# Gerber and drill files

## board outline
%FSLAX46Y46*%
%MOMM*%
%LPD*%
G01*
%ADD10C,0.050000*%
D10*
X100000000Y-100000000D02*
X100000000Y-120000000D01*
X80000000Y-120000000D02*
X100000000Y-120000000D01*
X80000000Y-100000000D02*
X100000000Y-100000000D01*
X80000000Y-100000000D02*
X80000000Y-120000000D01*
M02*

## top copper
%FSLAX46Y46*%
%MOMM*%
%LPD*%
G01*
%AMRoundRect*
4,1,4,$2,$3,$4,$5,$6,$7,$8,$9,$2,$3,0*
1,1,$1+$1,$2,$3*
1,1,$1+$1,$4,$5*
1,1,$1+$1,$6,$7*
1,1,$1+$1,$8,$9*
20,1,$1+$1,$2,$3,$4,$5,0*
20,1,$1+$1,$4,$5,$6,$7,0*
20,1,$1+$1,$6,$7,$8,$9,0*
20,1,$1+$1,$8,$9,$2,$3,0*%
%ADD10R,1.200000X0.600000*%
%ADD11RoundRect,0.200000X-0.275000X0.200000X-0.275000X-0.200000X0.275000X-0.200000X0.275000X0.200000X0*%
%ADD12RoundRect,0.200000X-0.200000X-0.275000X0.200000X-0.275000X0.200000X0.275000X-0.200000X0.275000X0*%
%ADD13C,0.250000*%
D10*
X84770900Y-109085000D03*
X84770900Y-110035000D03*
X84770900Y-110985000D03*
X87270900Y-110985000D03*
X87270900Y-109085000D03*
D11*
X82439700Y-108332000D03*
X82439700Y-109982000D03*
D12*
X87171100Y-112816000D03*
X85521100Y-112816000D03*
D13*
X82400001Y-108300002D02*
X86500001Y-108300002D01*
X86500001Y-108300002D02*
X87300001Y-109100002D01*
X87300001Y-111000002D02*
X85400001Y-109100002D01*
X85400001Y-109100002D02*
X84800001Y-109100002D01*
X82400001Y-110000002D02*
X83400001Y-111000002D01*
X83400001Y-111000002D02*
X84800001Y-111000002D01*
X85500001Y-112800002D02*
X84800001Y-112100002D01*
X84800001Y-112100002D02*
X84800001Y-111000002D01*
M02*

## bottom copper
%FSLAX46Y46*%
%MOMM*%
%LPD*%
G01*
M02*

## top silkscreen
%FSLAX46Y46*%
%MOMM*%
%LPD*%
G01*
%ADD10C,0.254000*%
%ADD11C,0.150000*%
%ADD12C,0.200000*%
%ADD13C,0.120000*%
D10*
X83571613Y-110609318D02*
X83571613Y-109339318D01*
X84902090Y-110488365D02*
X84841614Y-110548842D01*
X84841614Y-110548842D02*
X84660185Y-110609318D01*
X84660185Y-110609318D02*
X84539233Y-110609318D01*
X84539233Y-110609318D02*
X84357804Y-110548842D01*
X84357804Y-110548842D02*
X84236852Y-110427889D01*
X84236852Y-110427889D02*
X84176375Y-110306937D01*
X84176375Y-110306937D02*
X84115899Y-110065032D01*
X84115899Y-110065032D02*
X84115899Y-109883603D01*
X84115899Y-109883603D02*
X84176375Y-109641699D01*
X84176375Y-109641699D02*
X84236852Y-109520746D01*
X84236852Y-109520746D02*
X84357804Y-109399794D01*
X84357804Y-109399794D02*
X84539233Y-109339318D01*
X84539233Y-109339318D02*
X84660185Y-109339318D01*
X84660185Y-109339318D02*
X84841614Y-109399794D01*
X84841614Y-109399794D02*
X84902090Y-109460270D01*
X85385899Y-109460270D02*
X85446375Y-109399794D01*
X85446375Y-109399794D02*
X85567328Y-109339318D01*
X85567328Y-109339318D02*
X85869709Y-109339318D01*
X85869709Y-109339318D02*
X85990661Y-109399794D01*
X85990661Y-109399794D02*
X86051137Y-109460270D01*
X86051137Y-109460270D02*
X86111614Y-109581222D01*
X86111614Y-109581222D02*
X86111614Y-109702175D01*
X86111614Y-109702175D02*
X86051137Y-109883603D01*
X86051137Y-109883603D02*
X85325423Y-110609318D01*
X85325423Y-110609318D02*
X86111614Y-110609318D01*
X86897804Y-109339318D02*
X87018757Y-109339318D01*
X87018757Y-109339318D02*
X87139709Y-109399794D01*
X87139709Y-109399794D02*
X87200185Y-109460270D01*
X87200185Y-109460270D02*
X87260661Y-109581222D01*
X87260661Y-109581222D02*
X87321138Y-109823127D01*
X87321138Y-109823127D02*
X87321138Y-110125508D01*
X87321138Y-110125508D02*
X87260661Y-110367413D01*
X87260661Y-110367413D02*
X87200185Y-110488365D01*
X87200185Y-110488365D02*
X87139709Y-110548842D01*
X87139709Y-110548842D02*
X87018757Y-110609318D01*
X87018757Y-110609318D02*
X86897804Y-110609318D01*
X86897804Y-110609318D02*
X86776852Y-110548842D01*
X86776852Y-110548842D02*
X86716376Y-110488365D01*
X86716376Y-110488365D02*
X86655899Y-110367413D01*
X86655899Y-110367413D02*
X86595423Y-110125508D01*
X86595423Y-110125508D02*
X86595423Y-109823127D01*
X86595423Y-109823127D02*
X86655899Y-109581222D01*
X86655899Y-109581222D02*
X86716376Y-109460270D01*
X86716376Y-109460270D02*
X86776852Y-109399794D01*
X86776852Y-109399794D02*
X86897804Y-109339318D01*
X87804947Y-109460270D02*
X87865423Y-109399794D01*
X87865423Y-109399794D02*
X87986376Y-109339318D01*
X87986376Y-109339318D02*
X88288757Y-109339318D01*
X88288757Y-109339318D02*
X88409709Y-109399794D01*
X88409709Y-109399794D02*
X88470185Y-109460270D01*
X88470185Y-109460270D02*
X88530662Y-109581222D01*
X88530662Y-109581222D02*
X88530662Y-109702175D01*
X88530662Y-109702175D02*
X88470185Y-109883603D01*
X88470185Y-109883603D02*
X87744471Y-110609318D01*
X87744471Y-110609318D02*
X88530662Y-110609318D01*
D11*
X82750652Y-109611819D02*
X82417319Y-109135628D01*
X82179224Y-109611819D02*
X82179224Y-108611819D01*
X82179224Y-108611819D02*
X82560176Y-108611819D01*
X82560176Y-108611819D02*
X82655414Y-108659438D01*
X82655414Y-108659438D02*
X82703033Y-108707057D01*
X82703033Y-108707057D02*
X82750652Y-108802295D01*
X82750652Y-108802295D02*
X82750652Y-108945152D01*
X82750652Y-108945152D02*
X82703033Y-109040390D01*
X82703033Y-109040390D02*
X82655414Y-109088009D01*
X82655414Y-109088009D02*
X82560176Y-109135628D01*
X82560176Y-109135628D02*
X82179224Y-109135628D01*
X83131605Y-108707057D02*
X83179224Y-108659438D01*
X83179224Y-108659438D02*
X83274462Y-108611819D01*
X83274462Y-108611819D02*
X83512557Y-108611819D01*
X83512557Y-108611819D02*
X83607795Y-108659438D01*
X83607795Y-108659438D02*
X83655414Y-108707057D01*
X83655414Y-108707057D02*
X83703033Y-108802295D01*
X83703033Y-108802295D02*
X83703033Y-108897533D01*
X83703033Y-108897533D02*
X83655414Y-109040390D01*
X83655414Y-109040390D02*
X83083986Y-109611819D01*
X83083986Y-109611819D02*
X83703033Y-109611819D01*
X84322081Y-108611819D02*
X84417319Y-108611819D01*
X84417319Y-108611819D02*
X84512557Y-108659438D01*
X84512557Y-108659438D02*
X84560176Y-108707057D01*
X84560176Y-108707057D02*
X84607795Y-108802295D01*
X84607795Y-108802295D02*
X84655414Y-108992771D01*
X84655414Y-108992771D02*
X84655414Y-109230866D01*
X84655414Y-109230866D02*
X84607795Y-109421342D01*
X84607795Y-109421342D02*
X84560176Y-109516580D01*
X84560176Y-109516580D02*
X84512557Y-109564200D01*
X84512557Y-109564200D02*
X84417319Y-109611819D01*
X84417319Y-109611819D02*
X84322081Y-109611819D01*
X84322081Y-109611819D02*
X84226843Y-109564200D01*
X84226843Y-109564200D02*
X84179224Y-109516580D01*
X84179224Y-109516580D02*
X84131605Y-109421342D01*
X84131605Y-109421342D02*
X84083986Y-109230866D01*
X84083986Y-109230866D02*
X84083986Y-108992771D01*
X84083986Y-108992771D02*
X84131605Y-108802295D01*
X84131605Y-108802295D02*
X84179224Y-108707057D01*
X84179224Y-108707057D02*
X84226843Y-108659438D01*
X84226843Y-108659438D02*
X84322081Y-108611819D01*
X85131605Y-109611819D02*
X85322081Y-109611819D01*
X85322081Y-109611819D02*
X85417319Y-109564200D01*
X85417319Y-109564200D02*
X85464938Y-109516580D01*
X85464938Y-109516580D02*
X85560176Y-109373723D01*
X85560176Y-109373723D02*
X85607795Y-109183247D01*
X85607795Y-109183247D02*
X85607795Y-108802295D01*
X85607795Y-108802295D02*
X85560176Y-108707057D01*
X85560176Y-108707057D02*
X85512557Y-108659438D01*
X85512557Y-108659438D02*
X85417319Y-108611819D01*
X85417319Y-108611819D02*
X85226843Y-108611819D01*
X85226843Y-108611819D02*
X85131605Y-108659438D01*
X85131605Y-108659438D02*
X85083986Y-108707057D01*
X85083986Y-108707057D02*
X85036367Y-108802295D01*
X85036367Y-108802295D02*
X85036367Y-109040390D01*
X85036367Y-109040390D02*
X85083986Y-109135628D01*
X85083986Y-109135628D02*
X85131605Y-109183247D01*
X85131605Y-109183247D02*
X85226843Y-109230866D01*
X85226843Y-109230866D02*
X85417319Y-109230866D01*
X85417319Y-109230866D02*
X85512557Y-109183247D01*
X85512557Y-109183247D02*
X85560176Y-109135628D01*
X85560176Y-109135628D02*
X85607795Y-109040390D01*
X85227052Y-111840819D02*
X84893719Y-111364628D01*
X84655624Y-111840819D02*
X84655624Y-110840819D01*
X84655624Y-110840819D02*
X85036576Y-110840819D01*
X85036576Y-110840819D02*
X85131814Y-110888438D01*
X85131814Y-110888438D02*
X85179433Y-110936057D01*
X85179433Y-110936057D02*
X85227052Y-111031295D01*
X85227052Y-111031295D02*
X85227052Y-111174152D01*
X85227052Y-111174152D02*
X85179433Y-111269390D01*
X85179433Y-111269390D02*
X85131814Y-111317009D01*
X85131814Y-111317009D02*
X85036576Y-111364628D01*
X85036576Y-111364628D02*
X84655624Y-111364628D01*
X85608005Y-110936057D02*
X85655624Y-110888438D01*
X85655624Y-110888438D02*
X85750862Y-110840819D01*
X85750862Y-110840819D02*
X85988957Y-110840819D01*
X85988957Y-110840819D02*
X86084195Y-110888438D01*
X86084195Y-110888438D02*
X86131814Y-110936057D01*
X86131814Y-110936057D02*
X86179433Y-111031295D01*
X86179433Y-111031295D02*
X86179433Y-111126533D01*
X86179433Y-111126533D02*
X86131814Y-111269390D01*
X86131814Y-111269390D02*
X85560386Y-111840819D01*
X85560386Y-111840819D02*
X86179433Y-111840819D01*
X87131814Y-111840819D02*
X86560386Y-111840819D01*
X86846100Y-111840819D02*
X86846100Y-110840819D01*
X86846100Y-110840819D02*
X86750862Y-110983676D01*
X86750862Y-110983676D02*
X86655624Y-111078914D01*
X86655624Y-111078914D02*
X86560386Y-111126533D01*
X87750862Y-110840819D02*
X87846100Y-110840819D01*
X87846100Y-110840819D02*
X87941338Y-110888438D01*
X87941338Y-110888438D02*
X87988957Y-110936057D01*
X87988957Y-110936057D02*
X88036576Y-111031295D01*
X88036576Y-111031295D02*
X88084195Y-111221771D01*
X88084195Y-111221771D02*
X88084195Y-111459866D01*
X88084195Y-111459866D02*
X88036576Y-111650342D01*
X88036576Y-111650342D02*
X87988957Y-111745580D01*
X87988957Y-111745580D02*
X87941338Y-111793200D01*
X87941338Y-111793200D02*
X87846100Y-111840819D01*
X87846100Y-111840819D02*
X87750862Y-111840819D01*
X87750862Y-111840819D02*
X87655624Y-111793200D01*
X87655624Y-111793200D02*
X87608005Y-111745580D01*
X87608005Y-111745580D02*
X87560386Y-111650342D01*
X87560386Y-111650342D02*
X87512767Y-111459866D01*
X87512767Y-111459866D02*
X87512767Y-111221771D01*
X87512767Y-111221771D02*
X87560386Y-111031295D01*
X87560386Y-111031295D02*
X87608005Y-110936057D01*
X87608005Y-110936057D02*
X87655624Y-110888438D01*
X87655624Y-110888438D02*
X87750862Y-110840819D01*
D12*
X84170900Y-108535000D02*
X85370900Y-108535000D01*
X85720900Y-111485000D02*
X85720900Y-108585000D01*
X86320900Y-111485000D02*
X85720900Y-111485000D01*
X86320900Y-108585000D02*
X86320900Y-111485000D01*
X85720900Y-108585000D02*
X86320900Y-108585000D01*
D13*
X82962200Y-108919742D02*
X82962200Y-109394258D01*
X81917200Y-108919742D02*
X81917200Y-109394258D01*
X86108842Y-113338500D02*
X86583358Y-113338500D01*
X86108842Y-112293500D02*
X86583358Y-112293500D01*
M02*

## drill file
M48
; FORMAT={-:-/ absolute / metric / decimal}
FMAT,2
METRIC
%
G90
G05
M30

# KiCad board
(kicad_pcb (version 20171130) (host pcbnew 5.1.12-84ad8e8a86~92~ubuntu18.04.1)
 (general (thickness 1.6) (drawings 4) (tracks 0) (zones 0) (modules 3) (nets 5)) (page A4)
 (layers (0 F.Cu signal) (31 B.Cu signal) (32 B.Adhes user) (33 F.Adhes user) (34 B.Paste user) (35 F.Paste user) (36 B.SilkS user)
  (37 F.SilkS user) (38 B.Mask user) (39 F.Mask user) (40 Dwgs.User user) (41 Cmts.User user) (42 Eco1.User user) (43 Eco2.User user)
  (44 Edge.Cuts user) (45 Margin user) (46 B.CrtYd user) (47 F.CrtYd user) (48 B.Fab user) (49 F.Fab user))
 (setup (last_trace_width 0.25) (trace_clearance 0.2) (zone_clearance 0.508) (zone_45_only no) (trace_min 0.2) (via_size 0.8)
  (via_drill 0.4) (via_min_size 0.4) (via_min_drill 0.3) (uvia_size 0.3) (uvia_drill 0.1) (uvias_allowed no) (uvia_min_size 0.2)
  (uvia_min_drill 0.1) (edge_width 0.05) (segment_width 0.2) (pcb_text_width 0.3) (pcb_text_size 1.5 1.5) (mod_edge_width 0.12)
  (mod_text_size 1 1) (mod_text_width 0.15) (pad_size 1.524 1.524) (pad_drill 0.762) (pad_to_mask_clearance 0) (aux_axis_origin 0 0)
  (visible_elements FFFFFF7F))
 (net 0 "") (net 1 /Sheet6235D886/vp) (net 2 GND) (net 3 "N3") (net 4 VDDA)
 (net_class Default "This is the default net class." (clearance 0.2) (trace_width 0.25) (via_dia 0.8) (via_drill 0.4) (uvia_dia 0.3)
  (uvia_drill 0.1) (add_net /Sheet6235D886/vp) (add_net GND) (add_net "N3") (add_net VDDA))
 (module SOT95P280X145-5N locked (layer F.Cu) (at 86.020900 110.035000)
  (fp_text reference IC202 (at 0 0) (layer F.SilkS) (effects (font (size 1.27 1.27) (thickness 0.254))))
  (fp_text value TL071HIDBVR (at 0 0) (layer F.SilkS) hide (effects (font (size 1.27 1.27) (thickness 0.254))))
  (fp_line (start -1.85 -1.5) (end -0.65 -1.5) (layer F.SilkS) (width 0.2))
  (fp_line (start -0.3 1.45) (end -0.3 -1.45) (layer F.SilkS) (width 0.2))
  (fp_line (start 0.3 1.45) (end -0.3 1.45) (layer F.SilkS) (width 0.2))
  (fp_line (start 0.3 -1.45) (end 0.3 1.45) (layer F.SilkS) (width 0.2))
  (fp_line (start -0.3 -1.45) (end 0.3 -1.45) (layer F.SilkS) (width 0.2))
  (pad 1 smd rect (at -1.25 -0.95 90.000000) (size 0.6 1.2) (layers F.Cu F.Mask F.Paste) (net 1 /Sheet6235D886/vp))
  (pad 2 smd rect (at -1.25 0 90.000000) (size 0.6 1.2) (layers F.Cu F.Mask F.Paste) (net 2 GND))
  (pad 3 smd rect (at -1.25 0.95 90.000000) (size 0.6 1.2) (layers F.Cu F.Mask F.Paste) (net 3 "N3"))
  (pad 4 smd rect (at 1.25 0.95 90.000000) (size 0.6 1.2) (layers F.Cu F.Mask F.Paste) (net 1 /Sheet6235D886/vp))
  (pad 5 smd rect (at 1.25 -0.95 90.000000) (size 0.6 1.2) (layers F.Cu F.Mask F.Paste) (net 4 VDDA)))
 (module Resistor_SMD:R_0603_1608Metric (layer F.Cu) (at 82.439700 109.157000 270.000000)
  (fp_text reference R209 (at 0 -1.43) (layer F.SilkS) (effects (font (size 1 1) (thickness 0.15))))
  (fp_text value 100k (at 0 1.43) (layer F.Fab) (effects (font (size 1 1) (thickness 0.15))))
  (fp_line (start -0.237258 -0.5225) (end 0.237258 -0.5225) (layer F.SilkS) (width 0.12))
  (fp_line (start -0.237258 0.5225) (end 0.237258 0.5225) (layer F.SilkS) (width 0.12))
  (pad 1 smd roundrect (at -0.825 0 270.000000) (size 0.8 0.95) (layers F.Cu F.Mask F.Paste) (roundrect_rratio 0.25) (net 4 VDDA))
  (pad 2 smd roundrect (at 0.825 0 270.000000) (size 0.8 0.95) (layers F.Cu F.Mask F.Paste) (roundrect_rratio 0.25) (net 3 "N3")))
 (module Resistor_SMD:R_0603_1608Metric (layer F.Cu) (at 86.346100 112.816000)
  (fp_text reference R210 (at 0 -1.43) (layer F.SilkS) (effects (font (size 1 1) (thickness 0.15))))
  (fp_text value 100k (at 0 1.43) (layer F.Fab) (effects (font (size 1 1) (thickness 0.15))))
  (fp_line (start -0.237258 0.5225) (end 0.237258 0.5225) (layer F.SilkS) (width 0.12))
  (fp_line (start -0.237258 -0.5225) (end 0.237258 -0.5225) (layer F.SilkS) (width 0.12))
  (pad 2 smd roundrect (at 0.825 0) (size 0.8 0.95) (layers F.Cu F.Mask F.Paste) (roundrect_rratio 0.25) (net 2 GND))
  (pad 1 smd roundrect (at -0.825 0) (size 0.8 0.95) (layers F.Cu F.Mask F.Paste) (roundrect_rratio 0.25) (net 3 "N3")))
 (gr_line (start 100 100) (end 100 120) (layer Edge.Cuts) (width 0.05))
 (gr_line (start 80 120) (end 100 120) (layer Edge.Cuts) (width 0.05))
 (gr_line (start 80 100) (end 100 100) (layer Edge.Cuts) (width 0.05))
 (gr_line (start 80 100) (end 80 120) (layer Edge.Cuts) (width 0.05))
 (segment (start 82.400001 108.300002) (end 86.500001 108.300002) (width 0.250000) (layer F.Cu) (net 4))
 (segment (start 86.500001 108.300002) (end 87.300001 109.100002) (width 0.250000) (layer F.Cu) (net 4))
 (segment (start 87.300001 111.000002) (end 85.400001 109.100002) (width 0.250000) (layer F.Cu) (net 1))
 (segment (start 85.400001 109.100002) (end 84.800001 109.100002) (width 0.250000) (layer F.Cu) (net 1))
 (segment (start 82.400001 110.000002) (end 83.400001 111.000002) (width 0.250000) (layer F.Cu) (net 3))
 (segment (start 83.400001 111.000002) (end 84.800001 111.000002) (width 0.250000) (layer F.Cu) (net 3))
 (segment (start 85.500001 112.800002) (end 84.800001 112.100002) (width 0.250000) (layer F.Cu) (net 3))
 (segment (start 84.800001 112.100002) (end 84.800001 111.000002) (width 0.250000) (layer F.Cu) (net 3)))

